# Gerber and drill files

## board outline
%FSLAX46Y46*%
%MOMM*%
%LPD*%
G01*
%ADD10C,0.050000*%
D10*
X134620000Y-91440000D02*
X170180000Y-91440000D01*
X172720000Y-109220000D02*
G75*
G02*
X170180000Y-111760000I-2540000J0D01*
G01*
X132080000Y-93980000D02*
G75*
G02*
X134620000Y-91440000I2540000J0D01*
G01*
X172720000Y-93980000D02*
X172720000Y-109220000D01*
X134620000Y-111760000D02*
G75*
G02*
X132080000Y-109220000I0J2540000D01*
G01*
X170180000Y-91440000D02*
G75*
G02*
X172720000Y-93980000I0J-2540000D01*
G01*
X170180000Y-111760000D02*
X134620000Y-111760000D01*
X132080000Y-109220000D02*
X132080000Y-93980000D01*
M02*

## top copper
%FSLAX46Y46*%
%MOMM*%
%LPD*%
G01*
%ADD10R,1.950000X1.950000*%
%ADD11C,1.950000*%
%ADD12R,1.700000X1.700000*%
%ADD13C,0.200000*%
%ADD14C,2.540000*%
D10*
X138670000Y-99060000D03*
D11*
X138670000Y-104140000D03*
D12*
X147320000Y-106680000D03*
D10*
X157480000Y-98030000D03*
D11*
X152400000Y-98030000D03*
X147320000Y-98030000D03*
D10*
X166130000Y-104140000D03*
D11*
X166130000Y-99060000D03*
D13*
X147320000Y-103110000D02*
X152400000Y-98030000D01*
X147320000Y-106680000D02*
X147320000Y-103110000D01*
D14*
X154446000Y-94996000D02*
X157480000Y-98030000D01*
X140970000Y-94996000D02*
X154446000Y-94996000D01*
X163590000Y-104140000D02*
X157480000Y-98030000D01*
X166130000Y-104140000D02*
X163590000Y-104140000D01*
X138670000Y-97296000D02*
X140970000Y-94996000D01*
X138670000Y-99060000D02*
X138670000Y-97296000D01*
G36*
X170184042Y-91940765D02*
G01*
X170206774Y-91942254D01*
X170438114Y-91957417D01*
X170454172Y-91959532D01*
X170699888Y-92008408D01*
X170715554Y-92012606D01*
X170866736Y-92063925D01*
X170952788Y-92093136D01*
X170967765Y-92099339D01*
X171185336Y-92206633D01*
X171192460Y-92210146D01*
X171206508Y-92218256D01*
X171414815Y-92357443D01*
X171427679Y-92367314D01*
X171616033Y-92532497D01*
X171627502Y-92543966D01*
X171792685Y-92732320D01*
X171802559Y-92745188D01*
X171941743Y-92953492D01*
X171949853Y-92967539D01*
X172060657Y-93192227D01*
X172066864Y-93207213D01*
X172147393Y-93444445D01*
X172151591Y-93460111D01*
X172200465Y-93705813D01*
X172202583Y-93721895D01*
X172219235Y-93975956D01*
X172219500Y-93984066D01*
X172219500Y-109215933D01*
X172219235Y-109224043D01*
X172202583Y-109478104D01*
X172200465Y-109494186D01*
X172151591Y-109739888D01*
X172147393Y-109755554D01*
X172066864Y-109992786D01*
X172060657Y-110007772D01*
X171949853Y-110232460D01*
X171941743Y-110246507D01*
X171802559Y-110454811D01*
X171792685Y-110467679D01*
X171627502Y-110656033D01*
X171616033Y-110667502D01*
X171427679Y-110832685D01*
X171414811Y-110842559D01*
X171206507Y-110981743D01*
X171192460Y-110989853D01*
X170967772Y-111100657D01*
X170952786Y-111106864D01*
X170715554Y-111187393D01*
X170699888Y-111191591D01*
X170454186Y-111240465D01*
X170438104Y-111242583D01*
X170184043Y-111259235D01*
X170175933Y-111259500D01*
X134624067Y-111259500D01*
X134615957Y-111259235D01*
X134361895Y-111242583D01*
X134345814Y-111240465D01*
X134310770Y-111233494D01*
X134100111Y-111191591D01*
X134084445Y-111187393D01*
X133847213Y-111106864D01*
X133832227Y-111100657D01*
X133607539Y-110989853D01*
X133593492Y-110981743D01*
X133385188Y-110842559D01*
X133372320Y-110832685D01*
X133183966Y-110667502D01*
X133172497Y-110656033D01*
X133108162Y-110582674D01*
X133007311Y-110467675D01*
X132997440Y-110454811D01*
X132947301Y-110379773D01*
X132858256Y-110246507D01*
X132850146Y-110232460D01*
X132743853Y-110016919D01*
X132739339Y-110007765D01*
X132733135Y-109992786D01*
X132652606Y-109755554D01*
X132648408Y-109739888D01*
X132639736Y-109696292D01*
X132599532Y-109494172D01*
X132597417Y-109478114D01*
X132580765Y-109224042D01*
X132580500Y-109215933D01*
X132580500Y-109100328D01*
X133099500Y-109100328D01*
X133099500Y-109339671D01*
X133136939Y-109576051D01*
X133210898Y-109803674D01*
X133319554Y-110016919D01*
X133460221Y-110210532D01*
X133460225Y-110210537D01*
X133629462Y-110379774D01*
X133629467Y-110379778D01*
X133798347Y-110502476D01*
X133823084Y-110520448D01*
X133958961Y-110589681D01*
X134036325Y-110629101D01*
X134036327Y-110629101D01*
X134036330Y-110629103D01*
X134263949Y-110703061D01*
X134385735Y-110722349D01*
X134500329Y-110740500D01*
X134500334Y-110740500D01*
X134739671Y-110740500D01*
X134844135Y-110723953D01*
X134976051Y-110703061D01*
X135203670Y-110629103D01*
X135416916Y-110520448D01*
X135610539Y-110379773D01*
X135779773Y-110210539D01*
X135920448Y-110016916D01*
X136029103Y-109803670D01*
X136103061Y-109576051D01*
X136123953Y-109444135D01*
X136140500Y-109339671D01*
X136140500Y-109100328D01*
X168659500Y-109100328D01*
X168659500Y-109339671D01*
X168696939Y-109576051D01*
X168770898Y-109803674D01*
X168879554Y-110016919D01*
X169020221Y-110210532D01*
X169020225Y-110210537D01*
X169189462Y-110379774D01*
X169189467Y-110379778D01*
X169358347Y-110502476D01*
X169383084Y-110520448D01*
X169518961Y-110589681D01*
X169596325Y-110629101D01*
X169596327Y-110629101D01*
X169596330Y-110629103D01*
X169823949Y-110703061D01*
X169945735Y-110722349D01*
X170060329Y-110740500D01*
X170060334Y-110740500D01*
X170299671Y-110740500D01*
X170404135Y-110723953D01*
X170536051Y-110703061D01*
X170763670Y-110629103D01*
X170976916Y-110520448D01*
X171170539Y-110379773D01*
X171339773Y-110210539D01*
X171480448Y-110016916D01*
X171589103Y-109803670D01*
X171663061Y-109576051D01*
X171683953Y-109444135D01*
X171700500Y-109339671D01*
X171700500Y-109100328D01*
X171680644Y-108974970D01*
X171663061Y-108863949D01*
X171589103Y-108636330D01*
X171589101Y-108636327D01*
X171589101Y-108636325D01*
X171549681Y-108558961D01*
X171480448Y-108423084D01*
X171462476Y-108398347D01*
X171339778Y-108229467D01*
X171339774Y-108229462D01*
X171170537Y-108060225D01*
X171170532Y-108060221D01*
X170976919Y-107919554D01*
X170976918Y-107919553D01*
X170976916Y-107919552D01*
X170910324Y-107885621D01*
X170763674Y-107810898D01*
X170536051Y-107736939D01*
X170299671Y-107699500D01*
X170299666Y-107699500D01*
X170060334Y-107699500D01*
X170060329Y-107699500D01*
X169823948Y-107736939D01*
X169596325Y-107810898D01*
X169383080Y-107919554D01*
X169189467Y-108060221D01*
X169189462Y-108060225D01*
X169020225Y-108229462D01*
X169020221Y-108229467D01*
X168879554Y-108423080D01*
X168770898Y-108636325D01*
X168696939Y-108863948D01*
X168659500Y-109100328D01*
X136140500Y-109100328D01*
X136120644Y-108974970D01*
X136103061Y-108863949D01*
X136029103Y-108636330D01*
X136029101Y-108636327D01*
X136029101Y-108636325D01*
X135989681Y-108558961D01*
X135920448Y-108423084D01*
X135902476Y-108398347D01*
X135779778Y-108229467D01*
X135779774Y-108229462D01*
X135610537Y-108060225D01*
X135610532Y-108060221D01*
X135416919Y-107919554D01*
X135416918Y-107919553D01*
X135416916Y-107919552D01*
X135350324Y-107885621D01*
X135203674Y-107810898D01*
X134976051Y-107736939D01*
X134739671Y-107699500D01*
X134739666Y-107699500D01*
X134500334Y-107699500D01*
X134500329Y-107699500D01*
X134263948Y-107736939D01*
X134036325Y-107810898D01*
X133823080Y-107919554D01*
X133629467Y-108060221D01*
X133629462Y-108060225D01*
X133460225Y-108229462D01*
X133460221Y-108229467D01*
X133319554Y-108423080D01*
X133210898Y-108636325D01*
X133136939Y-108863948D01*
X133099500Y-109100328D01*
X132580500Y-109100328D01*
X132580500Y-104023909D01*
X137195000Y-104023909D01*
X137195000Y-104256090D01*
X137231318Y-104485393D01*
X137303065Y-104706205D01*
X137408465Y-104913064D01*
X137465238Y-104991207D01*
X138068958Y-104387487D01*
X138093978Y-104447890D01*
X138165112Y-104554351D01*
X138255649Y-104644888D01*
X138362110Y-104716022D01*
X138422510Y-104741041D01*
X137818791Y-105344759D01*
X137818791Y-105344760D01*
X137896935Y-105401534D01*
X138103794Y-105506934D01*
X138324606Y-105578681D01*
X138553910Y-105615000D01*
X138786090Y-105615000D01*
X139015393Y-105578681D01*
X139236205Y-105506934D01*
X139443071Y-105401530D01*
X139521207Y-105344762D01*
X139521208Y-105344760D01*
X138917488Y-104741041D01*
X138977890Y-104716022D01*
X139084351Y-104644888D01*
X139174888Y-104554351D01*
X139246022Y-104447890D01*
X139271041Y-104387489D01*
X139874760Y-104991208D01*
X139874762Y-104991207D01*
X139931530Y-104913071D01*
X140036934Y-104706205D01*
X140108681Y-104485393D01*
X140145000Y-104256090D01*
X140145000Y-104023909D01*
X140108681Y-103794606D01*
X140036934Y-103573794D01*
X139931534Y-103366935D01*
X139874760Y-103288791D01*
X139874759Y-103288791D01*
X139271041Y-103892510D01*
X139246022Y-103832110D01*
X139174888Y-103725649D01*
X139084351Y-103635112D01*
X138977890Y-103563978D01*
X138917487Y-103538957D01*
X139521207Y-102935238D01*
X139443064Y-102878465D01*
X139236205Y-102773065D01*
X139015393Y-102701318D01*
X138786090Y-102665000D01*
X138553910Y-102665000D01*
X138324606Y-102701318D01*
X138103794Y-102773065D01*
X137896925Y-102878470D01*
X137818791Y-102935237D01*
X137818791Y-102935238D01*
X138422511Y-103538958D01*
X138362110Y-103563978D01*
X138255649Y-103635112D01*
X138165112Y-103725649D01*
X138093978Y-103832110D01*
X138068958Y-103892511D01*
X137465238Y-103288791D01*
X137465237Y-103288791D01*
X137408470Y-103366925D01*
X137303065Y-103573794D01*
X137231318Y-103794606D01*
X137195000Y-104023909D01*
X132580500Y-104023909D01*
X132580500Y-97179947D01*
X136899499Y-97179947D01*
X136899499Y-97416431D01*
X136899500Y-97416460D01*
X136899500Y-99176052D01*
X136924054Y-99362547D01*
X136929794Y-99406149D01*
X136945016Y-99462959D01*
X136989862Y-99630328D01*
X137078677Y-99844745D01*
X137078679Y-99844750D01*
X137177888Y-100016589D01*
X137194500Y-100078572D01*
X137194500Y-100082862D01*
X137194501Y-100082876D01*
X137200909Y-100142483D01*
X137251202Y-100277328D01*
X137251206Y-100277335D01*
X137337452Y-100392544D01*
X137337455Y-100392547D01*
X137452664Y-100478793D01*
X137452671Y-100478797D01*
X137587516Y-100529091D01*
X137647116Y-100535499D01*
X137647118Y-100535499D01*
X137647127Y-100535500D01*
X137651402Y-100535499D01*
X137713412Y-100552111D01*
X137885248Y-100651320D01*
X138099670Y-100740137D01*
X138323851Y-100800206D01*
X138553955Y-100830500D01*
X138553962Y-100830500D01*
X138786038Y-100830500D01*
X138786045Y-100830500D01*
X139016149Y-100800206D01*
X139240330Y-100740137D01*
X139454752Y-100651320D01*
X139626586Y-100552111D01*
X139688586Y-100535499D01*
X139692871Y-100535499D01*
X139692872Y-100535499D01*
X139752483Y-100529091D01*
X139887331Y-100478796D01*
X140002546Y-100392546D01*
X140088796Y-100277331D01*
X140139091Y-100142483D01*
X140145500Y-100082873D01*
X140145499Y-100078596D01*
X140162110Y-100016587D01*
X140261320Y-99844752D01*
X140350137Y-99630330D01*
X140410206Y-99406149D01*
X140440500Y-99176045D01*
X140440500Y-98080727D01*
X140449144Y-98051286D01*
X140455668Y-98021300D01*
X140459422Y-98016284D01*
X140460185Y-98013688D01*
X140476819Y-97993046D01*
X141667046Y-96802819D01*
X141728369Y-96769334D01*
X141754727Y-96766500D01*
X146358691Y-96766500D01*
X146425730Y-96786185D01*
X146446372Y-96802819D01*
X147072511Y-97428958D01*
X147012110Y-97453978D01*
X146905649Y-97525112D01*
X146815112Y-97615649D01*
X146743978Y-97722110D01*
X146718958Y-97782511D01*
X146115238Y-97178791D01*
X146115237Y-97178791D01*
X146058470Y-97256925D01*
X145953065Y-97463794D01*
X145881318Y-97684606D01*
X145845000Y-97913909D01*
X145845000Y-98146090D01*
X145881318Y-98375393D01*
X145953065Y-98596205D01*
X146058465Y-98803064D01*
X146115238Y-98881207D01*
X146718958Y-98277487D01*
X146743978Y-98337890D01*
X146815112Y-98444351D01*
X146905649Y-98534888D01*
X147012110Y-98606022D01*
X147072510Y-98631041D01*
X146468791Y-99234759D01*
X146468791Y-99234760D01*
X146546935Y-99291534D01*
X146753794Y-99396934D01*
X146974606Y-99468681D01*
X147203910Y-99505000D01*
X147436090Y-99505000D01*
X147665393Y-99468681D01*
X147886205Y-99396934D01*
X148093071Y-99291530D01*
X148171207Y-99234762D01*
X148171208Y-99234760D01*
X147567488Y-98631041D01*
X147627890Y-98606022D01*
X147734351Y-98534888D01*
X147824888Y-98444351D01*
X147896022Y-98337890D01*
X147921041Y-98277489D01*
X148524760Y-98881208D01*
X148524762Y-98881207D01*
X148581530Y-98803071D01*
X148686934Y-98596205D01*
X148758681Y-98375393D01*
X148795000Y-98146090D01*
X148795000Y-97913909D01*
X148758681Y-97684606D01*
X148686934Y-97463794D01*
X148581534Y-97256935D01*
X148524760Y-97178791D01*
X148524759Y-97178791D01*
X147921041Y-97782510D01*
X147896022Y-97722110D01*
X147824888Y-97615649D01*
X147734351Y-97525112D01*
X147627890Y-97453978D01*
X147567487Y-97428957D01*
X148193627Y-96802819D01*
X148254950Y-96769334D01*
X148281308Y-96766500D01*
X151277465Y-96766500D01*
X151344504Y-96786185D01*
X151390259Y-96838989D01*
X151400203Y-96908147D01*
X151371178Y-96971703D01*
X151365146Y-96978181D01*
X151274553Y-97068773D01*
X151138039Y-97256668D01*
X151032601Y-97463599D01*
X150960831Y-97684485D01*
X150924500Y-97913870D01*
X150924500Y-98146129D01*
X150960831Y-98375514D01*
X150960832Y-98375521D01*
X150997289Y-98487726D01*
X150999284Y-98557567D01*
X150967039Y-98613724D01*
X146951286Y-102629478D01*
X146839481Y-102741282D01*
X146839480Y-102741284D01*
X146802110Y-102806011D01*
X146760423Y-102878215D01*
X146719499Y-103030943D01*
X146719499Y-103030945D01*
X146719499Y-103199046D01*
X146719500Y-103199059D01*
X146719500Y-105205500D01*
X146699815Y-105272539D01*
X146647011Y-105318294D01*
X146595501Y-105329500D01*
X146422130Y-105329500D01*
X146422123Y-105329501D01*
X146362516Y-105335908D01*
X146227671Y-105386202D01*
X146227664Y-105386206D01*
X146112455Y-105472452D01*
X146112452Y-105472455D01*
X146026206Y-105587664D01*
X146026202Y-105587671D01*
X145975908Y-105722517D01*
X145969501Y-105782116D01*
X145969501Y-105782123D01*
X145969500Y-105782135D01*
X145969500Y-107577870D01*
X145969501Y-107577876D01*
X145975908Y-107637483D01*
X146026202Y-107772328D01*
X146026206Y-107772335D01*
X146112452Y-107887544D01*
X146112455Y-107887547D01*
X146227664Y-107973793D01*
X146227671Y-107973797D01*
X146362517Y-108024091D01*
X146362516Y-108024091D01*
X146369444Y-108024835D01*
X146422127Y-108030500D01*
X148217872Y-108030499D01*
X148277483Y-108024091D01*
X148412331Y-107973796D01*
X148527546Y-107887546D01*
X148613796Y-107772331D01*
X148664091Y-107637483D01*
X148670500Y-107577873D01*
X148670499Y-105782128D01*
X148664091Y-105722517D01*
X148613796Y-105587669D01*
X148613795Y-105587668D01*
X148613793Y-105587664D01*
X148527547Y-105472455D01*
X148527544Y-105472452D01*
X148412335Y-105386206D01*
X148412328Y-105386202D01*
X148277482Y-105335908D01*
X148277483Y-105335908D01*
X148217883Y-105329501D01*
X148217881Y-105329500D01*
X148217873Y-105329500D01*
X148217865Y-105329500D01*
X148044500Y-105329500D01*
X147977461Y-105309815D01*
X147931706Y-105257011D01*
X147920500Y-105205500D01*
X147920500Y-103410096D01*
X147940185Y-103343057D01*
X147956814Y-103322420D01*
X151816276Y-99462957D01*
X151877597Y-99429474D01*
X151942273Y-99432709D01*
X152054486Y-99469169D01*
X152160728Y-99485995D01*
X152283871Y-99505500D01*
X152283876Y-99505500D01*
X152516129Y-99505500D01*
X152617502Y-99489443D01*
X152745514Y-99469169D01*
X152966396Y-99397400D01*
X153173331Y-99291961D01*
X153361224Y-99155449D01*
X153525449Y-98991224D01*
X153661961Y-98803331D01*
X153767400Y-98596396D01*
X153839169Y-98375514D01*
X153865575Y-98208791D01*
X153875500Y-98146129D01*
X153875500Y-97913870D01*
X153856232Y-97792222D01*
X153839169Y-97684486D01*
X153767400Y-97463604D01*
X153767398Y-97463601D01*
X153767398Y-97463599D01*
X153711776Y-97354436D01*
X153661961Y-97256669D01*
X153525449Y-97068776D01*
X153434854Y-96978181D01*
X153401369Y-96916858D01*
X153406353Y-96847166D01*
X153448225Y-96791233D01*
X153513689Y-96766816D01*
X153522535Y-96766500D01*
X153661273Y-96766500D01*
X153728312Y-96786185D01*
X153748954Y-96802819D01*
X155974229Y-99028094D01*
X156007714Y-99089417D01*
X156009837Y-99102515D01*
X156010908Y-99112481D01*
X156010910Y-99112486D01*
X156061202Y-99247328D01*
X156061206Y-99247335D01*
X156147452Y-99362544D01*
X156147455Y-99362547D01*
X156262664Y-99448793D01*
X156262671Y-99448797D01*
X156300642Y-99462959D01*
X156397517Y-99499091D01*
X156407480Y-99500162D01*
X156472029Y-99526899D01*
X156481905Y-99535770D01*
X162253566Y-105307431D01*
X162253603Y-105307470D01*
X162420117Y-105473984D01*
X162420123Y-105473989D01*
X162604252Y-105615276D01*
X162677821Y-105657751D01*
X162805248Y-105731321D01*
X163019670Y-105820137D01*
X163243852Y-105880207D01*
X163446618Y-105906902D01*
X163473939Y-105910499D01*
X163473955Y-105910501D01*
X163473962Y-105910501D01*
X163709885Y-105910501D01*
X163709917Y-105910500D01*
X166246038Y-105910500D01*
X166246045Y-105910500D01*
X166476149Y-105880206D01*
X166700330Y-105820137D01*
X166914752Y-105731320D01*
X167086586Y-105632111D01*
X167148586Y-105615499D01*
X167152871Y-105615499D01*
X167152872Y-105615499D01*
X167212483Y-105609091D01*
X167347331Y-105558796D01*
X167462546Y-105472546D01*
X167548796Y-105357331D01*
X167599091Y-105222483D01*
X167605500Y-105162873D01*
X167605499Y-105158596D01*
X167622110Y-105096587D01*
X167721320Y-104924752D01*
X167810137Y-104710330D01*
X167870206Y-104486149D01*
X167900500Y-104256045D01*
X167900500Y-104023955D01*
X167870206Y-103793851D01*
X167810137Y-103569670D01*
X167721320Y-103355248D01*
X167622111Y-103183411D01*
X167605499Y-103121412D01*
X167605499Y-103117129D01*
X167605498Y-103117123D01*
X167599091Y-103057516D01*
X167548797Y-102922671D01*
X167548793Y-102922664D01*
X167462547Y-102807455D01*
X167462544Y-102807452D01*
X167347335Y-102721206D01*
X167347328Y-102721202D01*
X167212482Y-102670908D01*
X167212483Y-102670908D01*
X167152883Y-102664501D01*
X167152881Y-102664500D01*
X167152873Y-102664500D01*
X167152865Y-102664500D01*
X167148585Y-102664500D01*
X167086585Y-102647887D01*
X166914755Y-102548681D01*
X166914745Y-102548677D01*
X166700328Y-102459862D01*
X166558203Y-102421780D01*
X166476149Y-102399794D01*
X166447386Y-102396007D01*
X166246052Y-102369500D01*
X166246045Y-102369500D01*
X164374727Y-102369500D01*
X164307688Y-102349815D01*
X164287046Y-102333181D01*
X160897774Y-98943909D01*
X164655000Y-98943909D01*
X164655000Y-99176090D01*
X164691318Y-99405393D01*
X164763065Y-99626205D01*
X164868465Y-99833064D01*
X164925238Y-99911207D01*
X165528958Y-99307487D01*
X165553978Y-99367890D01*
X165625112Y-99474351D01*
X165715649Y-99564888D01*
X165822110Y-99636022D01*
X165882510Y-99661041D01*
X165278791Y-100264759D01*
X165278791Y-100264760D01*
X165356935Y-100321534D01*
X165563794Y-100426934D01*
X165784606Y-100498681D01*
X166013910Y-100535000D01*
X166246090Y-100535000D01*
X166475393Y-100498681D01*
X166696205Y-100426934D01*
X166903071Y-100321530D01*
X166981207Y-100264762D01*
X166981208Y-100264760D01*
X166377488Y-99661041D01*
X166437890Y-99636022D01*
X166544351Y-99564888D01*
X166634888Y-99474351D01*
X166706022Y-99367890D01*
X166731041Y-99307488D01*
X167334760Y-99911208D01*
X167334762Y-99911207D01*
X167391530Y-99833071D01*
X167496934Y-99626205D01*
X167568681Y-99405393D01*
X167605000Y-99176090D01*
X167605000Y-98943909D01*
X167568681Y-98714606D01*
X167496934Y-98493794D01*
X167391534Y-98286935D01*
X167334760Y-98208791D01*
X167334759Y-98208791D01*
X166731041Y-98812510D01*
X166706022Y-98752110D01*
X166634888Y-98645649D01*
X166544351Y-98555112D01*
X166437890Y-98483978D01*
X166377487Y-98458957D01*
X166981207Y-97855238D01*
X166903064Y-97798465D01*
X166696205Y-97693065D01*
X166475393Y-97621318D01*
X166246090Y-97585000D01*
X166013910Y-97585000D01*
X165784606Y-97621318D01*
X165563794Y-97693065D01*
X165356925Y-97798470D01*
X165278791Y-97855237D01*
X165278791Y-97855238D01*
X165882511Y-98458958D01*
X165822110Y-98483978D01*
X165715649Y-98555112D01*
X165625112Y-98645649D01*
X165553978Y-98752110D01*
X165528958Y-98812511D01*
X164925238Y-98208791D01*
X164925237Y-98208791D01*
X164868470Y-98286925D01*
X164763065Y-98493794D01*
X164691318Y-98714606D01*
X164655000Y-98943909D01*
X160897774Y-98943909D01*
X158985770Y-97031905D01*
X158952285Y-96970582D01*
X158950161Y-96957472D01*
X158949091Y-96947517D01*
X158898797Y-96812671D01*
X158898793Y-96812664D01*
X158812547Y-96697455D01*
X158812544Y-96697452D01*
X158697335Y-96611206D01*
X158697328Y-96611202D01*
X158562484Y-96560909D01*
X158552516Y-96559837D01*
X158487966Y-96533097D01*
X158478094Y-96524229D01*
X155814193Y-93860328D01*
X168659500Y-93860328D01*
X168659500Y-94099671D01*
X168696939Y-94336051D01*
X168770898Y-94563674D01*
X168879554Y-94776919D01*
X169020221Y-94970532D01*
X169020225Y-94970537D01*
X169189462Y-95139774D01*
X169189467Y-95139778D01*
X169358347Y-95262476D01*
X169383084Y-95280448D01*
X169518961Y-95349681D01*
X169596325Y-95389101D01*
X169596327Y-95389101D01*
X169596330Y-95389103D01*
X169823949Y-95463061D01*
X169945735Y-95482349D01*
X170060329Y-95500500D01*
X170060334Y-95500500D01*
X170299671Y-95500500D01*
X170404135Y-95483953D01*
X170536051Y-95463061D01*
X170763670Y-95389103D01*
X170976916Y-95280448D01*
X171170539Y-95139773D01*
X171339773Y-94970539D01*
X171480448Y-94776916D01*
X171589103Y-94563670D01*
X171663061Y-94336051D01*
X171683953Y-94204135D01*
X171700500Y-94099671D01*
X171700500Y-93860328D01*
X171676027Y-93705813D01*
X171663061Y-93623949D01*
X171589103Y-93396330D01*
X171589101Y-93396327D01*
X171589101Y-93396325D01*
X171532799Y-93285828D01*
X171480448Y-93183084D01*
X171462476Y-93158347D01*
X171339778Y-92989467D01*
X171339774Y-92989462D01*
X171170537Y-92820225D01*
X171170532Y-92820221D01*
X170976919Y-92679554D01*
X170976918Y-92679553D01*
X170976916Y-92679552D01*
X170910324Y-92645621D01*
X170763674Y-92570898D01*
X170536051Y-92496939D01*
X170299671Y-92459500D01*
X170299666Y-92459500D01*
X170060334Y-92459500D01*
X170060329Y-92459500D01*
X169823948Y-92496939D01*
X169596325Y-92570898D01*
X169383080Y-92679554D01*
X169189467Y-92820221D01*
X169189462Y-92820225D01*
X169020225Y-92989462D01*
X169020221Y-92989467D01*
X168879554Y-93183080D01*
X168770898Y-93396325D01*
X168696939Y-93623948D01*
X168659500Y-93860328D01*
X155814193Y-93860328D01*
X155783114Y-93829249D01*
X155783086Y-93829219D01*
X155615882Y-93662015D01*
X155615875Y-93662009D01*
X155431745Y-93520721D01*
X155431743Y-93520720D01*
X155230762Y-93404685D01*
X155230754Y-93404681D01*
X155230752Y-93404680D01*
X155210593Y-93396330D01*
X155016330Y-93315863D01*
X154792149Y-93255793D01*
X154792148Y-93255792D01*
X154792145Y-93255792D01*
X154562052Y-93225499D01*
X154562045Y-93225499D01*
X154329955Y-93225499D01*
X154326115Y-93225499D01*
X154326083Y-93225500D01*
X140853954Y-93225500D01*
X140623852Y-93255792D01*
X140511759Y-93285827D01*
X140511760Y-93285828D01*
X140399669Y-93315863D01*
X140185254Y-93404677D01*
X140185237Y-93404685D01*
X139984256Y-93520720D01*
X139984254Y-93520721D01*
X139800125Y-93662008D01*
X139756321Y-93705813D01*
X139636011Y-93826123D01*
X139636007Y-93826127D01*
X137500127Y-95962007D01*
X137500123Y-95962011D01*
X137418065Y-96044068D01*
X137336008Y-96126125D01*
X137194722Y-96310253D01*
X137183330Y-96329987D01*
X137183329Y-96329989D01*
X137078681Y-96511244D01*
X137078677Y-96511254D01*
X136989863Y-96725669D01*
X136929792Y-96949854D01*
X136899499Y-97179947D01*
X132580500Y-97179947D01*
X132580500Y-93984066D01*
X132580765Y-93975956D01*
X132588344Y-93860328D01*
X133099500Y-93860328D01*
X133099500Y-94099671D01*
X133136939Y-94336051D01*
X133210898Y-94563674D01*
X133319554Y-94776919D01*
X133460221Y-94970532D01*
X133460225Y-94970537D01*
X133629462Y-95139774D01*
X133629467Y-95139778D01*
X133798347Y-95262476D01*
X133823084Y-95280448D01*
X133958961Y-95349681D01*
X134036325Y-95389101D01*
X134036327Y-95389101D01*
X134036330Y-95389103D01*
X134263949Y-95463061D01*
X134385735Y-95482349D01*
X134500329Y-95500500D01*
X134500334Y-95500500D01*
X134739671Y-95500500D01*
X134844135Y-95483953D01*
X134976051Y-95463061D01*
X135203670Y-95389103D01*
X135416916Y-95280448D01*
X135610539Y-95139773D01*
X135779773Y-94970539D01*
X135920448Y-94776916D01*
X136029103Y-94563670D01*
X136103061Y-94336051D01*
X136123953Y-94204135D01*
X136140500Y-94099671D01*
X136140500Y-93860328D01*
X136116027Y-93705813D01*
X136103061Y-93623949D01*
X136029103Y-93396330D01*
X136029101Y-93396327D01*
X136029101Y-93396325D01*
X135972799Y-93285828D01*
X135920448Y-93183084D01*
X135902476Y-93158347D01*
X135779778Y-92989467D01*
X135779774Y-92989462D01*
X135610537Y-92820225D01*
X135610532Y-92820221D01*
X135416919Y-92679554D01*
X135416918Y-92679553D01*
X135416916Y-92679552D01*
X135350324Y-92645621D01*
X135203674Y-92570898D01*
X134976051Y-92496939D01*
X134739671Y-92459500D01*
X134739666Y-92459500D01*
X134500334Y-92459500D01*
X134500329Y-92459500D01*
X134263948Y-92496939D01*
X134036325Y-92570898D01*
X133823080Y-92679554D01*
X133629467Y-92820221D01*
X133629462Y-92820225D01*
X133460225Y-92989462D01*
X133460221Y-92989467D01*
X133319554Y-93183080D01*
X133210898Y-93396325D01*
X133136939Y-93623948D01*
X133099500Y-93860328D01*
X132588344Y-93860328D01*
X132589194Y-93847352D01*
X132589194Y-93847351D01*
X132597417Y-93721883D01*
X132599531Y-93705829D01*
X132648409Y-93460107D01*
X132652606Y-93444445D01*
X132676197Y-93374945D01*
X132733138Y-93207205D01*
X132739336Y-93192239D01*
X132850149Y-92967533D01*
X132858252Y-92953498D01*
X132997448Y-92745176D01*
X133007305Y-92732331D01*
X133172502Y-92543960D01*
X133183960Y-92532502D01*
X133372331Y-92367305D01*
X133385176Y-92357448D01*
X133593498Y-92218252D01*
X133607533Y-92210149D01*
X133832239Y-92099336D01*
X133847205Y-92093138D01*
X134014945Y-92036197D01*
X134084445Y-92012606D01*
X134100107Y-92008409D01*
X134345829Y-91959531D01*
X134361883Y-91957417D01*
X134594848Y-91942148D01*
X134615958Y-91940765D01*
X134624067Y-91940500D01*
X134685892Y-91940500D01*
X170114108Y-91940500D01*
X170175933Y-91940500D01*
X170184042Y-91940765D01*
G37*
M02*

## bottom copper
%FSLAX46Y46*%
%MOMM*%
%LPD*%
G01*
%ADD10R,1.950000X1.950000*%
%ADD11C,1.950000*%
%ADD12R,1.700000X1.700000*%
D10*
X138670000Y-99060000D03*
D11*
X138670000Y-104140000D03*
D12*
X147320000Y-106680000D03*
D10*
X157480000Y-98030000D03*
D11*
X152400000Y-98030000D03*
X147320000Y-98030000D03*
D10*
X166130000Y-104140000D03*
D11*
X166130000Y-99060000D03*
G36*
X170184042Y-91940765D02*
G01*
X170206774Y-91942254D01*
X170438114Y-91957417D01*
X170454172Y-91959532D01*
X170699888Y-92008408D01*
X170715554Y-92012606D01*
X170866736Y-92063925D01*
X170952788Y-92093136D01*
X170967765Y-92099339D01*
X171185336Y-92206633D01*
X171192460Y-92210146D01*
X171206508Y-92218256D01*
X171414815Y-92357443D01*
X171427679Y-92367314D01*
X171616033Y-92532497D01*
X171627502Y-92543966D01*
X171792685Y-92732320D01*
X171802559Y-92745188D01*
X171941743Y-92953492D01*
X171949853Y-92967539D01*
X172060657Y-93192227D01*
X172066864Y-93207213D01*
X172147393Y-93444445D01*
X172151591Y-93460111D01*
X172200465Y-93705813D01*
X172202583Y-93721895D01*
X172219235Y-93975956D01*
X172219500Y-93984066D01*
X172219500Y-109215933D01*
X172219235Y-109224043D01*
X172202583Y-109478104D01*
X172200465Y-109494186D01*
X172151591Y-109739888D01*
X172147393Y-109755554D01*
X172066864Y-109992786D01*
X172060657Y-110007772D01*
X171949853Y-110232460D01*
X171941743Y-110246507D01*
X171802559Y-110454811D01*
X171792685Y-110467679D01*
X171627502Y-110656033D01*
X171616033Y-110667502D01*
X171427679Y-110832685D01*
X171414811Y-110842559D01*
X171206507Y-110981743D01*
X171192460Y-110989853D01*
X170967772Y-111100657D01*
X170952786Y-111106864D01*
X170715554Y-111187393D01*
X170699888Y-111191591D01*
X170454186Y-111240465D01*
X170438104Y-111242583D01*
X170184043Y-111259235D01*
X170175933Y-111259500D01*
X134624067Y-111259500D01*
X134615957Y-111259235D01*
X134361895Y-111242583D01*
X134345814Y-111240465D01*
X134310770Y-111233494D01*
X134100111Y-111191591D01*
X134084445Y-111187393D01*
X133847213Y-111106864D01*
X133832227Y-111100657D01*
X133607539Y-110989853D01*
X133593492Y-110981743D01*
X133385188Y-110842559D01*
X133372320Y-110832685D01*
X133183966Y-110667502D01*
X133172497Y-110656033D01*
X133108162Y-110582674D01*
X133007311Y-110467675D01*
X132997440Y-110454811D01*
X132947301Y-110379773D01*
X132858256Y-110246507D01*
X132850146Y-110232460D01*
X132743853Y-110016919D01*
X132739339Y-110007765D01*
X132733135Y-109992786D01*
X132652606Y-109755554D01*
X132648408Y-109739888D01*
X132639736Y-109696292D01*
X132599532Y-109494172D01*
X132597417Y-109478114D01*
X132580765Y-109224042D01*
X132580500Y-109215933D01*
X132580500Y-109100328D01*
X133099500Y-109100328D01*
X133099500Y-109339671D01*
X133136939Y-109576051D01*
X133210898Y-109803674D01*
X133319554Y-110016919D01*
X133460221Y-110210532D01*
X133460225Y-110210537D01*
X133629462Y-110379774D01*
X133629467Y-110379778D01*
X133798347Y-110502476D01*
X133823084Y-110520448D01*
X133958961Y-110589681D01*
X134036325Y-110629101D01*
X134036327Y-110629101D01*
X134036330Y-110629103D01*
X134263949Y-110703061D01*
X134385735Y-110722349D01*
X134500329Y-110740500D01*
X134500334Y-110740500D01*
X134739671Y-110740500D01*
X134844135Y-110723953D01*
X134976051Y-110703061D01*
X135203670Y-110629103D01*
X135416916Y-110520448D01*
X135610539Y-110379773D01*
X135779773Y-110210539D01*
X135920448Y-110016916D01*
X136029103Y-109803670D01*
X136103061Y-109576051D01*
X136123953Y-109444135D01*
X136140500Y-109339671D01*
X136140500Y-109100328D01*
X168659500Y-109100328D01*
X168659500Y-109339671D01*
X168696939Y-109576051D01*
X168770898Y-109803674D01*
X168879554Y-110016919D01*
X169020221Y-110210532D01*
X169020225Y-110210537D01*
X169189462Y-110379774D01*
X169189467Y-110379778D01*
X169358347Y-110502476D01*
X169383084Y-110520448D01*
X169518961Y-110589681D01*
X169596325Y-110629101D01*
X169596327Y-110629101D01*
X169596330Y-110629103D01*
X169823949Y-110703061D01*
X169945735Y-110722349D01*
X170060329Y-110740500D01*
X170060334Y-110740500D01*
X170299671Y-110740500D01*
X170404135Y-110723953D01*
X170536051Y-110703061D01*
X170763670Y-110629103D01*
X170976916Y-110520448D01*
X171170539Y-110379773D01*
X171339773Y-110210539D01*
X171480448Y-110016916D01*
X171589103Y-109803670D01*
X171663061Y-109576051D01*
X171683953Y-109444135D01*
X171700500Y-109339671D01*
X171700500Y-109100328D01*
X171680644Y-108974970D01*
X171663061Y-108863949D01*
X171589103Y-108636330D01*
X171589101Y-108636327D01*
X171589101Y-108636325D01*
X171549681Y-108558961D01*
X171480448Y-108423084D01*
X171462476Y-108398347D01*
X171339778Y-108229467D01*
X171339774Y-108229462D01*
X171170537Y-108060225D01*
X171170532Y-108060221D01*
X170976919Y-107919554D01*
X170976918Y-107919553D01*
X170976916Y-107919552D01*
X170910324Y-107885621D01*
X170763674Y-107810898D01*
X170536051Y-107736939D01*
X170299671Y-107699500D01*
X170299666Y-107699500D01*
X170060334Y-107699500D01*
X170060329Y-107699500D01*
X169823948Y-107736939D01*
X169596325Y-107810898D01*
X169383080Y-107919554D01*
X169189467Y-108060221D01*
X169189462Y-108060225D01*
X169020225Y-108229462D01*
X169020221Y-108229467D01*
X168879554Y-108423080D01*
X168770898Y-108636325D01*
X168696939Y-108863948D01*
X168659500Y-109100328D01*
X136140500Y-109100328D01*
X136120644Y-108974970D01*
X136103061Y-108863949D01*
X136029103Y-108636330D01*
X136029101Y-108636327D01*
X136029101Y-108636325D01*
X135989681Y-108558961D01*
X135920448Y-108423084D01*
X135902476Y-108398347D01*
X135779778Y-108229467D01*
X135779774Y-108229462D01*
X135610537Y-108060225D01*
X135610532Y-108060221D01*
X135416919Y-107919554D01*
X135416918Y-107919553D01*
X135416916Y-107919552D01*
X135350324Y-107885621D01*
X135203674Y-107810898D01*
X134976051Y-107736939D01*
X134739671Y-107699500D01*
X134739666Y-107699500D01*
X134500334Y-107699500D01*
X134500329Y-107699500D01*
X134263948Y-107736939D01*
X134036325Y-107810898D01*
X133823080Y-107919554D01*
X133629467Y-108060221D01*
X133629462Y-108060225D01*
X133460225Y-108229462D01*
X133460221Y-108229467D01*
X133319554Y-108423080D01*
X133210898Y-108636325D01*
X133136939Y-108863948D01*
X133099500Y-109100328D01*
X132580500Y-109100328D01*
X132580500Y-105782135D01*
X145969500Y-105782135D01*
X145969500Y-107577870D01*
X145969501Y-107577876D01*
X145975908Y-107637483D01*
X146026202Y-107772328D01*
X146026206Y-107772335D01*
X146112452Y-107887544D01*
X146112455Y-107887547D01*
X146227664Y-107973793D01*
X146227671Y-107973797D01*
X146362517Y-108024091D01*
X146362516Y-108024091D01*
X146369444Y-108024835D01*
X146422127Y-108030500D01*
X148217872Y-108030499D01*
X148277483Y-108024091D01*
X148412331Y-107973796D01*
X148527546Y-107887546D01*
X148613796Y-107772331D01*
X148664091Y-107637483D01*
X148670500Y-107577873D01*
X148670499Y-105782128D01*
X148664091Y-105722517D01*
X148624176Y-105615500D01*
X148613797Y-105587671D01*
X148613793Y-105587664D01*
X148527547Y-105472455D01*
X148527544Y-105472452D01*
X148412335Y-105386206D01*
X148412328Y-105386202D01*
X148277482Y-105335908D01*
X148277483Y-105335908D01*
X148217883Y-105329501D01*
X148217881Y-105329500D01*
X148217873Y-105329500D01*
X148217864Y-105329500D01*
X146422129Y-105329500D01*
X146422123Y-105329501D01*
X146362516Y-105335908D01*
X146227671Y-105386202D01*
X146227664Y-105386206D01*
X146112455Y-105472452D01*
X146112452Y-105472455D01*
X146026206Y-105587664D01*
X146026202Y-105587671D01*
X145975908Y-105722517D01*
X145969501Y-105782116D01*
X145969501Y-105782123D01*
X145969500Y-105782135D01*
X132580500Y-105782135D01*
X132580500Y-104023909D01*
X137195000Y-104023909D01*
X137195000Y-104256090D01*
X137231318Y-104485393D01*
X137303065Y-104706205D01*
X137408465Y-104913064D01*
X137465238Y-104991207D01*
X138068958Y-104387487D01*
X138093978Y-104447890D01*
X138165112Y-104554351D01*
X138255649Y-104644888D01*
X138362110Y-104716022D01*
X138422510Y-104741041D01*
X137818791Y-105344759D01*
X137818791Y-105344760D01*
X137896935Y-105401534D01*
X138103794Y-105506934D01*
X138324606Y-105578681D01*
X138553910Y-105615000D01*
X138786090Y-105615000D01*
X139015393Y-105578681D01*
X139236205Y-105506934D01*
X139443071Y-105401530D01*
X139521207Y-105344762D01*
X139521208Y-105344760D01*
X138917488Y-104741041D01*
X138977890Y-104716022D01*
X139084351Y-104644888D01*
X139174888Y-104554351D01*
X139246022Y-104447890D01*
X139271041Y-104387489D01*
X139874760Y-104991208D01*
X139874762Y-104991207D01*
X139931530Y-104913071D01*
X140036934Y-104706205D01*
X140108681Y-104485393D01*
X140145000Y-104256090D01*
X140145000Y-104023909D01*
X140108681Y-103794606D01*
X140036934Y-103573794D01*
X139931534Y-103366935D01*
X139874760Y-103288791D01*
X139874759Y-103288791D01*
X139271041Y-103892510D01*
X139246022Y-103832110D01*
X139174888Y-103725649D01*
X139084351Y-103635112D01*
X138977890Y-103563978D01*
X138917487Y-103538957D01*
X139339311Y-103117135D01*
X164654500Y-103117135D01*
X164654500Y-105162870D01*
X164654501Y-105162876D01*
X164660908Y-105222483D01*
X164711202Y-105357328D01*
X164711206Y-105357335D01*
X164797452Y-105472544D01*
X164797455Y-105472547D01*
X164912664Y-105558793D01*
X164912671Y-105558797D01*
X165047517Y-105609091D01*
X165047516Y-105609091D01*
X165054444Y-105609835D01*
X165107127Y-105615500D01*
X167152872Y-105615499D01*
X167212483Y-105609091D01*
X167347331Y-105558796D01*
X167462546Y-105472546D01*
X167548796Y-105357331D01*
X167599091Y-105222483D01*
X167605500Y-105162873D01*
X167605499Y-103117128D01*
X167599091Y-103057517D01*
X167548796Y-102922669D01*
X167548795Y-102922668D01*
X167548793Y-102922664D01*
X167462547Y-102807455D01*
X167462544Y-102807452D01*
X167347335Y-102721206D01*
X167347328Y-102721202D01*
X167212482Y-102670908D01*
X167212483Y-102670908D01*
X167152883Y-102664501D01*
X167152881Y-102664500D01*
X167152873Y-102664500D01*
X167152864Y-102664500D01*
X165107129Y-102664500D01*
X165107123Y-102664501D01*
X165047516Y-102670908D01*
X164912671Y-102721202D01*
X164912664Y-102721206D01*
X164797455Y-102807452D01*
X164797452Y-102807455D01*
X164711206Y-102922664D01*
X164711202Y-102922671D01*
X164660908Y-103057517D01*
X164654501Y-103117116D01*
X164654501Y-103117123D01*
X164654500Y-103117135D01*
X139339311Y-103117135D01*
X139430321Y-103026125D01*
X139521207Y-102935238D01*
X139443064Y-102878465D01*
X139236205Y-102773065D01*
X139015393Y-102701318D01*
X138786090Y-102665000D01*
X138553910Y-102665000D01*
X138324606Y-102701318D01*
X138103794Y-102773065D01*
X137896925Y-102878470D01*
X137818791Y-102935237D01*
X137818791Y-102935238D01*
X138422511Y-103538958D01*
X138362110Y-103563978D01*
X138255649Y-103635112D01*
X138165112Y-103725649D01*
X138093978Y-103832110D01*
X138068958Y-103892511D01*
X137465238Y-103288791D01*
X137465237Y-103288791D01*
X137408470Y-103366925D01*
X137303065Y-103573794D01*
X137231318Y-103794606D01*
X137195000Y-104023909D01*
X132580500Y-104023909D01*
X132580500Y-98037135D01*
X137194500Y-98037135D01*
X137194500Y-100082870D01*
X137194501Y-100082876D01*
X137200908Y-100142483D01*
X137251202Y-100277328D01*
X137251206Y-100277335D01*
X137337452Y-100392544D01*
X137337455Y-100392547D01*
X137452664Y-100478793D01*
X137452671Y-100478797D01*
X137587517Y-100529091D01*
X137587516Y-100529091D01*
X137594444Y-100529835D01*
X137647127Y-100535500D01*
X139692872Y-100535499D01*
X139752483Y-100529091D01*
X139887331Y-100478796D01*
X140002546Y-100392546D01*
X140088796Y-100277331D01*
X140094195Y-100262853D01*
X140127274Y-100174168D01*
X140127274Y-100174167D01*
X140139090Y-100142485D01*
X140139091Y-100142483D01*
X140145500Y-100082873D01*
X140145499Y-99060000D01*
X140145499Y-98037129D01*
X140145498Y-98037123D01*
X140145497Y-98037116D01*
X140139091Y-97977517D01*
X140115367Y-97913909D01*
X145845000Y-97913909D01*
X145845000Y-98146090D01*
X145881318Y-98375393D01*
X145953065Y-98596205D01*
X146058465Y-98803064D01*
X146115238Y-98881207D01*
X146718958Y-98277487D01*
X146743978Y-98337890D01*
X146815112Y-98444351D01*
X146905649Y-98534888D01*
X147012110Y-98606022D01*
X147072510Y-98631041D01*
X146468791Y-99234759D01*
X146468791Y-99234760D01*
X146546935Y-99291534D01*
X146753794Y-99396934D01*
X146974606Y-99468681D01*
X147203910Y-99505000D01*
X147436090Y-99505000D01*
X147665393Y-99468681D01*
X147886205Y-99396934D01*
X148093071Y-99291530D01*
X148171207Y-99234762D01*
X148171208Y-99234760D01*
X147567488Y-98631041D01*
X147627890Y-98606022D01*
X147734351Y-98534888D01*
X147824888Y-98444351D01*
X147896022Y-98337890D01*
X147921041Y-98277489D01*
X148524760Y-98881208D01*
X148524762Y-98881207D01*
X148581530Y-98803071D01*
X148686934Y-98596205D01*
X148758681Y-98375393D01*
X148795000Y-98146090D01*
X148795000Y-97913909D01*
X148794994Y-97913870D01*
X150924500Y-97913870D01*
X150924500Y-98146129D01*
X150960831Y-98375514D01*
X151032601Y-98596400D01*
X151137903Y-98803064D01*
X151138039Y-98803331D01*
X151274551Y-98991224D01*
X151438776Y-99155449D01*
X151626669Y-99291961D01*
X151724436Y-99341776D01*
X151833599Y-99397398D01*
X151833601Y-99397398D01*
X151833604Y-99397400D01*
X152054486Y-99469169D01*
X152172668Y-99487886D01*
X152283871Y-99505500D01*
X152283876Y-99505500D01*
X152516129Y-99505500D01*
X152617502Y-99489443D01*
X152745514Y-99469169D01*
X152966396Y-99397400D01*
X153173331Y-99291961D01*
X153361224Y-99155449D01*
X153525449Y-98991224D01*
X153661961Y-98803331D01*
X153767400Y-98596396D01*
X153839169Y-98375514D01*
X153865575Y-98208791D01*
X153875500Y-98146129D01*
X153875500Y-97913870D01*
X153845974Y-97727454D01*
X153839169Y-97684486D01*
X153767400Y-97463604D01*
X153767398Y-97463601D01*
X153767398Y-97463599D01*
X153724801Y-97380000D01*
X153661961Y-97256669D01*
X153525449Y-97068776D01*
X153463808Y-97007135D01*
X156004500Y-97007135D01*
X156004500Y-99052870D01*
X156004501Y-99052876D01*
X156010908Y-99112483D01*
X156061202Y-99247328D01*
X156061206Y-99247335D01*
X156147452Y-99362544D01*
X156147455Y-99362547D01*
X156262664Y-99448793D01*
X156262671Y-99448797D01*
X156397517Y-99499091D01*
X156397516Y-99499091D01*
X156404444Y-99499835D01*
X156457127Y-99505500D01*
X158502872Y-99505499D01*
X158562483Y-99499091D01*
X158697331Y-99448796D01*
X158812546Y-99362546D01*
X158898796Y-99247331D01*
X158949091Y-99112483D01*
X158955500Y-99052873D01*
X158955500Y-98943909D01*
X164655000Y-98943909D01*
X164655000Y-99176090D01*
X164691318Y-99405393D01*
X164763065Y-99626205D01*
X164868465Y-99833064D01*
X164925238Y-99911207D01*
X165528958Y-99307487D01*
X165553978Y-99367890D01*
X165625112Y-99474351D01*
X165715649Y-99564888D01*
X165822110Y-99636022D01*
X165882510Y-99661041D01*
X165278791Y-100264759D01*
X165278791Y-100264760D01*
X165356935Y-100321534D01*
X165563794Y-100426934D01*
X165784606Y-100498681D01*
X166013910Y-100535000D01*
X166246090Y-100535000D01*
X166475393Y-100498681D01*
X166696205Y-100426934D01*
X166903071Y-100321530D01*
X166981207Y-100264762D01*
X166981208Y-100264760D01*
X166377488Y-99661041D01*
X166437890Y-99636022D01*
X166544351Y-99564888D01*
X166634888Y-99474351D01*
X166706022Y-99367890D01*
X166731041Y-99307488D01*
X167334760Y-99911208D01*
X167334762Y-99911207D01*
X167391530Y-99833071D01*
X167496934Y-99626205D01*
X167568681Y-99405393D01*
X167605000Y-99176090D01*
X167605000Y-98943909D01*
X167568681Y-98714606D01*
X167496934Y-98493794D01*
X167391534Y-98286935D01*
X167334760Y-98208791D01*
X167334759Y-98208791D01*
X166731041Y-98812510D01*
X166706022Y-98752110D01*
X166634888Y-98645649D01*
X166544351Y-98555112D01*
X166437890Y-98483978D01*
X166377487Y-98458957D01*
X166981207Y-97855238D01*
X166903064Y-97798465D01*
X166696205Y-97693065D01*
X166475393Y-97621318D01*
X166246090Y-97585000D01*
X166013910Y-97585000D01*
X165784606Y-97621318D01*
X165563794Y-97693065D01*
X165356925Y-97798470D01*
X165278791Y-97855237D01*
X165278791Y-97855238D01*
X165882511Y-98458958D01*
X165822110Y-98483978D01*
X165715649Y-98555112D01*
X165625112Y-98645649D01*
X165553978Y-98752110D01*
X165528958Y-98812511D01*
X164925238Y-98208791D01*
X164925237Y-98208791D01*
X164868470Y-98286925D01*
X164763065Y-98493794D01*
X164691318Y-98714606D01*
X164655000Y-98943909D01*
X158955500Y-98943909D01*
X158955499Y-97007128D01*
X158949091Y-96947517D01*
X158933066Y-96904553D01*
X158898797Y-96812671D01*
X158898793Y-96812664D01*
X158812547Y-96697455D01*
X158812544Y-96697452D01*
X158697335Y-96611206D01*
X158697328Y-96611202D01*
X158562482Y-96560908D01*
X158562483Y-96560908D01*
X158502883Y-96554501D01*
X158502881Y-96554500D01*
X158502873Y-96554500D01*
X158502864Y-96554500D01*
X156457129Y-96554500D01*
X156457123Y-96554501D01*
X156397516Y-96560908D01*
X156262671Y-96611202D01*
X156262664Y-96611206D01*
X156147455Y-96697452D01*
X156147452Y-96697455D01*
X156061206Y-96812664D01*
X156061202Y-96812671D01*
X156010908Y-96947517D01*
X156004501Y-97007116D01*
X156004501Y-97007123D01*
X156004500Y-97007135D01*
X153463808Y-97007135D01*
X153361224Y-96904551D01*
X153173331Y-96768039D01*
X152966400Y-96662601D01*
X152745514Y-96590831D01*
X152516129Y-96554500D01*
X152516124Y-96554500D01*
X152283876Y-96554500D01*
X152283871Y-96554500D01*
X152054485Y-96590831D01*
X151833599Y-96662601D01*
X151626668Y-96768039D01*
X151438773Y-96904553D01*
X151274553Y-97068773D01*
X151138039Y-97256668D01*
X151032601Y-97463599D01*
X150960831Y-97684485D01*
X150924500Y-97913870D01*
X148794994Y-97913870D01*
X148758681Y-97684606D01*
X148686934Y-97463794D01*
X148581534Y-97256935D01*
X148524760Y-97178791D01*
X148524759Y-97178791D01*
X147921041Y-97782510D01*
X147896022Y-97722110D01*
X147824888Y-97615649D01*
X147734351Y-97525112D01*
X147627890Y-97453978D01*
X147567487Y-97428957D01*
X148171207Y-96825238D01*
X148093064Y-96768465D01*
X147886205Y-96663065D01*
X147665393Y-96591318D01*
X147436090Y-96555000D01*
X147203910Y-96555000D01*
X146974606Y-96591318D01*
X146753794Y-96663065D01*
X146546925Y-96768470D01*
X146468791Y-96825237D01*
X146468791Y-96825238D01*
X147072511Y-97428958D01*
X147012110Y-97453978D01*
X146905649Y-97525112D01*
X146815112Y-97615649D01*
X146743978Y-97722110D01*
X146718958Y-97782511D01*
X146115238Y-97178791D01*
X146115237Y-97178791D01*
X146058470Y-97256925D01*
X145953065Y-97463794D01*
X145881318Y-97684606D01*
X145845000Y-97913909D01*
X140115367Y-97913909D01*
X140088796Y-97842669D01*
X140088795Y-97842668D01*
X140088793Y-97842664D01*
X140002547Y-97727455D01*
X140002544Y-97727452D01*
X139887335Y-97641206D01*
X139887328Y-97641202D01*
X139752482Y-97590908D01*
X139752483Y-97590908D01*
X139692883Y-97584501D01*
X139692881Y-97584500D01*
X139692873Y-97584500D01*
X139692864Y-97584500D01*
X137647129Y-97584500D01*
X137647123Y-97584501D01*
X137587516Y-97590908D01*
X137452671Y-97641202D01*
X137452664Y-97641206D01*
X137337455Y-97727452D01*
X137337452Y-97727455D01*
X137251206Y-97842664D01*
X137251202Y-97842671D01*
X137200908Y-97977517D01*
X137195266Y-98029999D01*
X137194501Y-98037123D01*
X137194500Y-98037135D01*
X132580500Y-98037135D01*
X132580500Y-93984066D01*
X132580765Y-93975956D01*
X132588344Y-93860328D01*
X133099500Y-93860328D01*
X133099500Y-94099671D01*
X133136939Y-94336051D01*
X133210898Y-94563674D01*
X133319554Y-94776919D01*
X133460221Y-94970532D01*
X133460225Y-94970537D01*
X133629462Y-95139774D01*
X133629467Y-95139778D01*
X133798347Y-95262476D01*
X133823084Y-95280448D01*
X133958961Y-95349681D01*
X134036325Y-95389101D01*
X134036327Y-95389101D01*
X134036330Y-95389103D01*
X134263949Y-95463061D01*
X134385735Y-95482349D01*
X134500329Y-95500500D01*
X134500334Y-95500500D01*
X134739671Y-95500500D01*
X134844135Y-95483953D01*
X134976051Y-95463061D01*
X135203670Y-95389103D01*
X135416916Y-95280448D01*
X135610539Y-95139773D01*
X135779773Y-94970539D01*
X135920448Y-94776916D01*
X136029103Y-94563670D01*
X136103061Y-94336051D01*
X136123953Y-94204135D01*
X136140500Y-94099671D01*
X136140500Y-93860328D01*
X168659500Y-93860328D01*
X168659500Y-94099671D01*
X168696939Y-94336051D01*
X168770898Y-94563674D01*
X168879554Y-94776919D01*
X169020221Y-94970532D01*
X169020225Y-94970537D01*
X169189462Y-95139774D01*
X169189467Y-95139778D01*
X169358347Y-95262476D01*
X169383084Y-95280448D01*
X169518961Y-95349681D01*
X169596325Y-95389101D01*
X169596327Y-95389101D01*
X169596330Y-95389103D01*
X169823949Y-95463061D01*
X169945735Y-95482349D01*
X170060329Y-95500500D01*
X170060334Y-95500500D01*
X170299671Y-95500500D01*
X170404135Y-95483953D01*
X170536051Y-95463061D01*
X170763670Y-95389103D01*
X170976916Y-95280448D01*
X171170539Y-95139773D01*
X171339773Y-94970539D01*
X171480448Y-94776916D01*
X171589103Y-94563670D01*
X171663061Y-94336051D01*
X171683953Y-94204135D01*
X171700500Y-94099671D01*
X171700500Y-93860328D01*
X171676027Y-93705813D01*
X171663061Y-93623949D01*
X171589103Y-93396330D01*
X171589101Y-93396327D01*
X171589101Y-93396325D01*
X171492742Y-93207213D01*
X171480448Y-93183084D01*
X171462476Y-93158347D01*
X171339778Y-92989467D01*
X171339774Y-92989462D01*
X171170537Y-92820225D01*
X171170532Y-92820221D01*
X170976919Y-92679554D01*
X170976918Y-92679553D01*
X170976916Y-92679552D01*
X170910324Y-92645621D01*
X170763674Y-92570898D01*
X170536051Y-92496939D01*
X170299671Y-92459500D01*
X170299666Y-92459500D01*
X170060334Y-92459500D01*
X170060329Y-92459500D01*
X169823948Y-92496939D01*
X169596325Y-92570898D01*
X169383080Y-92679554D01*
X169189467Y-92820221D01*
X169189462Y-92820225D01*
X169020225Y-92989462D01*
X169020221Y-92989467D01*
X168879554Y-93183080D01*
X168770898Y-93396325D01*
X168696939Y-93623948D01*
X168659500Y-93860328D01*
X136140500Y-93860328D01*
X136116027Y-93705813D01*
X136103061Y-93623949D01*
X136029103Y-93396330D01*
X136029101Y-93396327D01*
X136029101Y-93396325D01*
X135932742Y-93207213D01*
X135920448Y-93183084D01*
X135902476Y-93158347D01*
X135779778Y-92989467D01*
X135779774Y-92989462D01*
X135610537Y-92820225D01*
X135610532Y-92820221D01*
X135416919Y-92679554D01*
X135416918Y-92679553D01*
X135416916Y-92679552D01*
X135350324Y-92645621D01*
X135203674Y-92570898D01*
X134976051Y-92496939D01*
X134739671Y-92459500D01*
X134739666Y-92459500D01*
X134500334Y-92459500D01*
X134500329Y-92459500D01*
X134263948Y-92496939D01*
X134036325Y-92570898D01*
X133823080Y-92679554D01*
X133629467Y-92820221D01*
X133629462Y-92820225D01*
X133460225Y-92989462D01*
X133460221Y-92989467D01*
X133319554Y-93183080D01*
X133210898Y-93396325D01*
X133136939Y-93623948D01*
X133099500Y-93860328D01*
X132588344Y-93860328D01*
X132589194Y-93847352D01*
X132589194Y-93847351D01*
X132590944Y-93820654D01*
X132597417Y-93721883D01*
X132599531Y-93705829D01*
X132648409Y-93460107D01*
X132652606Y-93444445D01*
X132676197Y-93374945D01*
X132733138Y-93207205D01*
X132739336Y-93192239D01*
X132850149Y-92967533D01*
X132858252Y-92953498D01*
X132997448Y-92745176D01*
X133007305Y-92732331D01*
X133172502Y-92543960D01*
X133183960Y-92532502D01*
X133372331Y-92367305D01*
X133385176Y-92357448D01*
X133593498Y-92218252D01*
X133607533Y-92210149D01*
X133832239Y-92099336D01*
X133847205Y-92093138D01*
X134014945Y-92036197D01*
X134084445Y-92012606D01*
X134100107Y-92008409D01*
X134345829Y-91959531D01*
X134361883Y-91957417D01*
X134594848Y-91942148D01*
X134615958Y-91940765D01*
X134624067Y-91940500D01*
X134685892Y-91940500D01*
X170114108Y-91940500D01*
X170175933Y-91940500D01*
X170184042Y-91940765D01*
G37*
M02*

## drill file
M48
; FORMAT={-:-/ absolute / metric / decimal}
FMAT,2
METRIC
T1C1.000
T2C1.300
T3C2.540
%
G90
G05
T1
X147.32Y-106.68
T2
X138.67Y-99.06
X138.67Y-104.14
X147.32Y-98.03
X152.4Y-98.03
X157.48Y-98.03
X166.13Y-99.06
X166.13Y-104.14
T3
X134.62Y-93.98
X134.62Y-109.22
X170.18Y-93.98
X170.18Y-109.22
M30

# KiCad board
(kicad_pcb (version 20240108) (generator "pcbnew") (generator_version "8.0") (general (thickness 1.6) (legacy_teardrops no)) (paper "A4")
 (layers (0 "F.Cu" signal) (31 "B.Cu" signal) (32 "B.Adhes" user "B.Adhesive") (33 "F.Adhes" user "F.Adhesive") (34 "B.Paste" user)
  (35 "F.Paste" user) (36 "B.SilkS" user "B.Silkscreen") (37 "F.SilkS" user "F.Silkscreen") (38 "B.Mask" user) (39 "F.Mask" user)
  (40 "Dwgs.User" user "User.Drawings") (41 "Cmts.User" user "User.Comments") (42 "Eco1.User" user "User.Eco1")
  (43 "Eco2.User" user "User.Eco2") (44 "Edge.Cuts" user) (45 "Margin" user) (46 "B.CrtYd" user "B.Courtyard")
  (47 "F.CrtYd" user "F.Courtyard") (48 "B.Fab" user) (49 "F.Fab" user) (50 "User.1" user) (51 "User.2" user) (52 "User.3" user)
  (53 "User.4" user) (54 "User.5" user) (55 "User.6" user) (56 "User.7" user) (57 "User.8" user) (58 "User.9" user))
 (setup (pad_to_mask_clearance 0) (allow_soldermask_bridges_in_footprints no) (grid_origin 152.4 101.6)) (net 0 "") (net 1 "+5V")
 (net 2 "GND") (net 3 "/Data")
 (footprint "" (layer "F.Cu") (at 134.62 109.22)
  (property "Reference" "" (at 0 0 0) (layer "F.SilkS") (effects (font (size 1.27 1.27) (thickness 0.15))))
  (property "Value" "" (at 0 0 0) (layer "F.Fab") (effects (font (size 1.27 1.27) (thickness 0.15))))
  (pad "" np_thru_hole circle (at 0 0) (size 2.5 2.5) (drill 2.54) (layers "F&B.Cu" "*.Mask")))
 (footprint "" (layer "F.Cu") (at 170.18 93.98)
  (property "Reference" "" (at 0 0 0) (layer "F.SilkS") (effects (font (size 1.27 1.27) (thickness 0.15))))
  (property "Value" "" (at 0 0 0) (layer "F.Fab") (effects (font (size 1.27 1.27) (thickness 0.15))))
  (pad "" np_thru_hole circle (at 0 0) (size 2.5 2.5) (drill 2.54) (layers "F&B.Cu" "*.Mask")))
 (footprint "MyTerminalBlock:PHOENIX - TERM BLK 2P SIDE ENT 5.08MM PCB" (layer "F.Cu") (at 134.62 96.52 -90)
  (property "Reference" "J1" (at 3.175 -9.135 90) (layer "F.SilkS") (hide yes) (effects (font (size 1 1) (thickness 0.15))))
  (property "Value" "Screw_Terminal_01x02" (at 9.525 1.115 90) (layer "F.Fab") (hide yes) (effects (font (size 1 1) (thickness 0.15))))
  (pad "1" thru_hole rect (at 2.54 -4.05 270) (size 1.95 1.95) (drill 1.3) (layers "*.Cu" "*.Mask") (remove_unused_layers no) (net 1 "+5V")
   (solder_mask_margin 0.102))
  (pad "2" thru_hole circle (at 7.62 -4.05 270) (size 1.95 1.95) (drill 1.3) (layers "*.Cu" "*.Mask") (remove_unused_layers no)
   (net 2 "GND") (solder_mask_margin 0.102)))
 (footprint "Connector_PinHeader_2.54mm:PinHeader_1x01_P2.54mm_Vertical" (layer "F.Cu") (at 147.32 106.68 -90)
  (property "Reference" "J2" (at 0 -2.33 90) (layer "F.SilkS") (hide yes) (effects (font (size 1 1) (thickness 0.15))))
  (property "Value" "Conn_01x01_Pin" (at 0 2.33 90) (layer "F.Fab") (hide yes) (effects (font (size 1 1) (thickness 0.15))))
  (pad "1" thru_hole rect (at 0 0 270) (size 1.7 1.7) (drill 1) (layers "*.Cu" "*.Mask") (remove_unused_layers no) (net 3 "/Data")))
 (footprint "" (layer "F.Cu") (at 134.62 93.98)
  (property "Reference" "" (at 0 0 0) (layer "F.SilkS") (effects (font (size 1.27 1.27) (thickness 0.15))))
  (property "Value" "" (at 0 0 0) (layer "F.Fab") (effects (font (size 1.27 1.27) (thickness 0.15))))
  (pad "" np_thru_hole circle (at 0 0) (size 2.5 2.5) (drill 2.54) (layers "F&B.Cu" "*.Mask")))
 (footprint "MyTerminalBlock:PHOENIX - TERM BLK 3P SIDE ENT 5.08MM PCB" (layer "F.Cu") (at 160.02 93.98 180)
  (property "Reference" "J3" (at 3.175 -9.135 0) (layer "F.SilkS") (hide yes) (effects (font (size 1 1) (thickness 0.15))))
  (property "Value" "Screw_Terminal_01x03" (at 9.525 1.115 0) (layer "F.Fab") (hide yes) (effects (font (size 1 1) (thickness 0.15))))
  (pad "1" thru_hole rect (at 2.54 -4.05 180) (size 1.95 1.95) (drill 1.3) (layers "*.Cu" "*.Mask") (remove_unused_layers no) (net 1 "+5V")
   (solder_mask_margin 0.102))
  (pad "2" thru_hole circle (at 7.62 -4.05 180) (size 1.95 1.95) (drill 1.3) (layers "*.Cu" "*.Mask") (remove_unused_layers no)
   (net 3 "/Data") (solder_mask_margin 0.102))
  (pad "3" thru_hole circle (at 12.7 -4.05 180) (size 1.95 1.95) (drill 1.3) (layers "*.Cu" "*.Mask") (remove_unused_layers no)
   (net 2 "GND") (solder_mask_margin 0.102)))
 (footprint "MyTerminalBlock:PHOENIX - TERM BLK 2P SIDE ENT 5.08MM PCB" (layer "F.Cu") (at 170.18 106.68 90)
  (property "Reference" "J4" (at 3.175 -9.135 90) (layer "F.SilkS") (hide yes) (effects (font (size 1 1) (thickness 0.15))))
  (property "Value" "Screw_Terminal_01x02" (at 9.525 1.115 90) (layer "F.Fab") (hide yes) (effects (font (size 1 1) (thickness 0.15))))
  (pad "1" thru_hole rect (at 2.54 -4.05 90) (size 1.95 1.95) (drill 1.3) (layers "*.Cu" "*.Mask") (remove_unused_layers no) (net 1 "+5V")
   (solder_mask_margin 0.102))
  (pad "2" thru_hole circle (at 7.62 -4.05 90) (size 1.95 1.95) (drill 1.3) (layers "*.Cu" "*.Mask") (remove_unused_layers no) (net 2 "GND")
   (solder_mask_margin 0.102)))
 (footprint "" (layer "F.Cu") (at 170.18 109.22)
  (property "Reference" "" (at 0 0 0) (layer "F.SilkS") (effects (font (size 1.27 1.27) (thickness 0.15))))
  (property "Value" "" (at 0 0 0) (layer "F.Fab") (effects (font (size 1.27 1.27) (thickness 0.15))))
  (pad "" np_thru_hole circle (at 0 0) (size 2.5 2.5) (drill 2.54) (layers "F&B.Cu" "*.Mask")))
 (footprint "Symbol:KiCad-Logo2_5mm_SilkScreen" (layer "B.Cu") (at 156.845 106.045 180)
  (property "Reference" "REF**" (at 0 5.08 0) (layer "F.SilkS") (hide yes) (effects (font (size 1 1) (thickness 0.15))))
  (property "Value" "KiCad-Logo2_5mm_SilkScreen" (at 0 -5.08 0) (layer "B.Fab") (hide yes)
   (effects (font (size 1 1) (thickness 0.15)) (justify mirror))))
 (gr_line (start 134.62 91.44) (end 170.18 91.44) (stroke (width 0.05) (type default)) (layer "Edge.Cuts"))
 (gr_arc (start 172.72 109.22) (mid 171.976051 111.016051) (end 170.18 111.76) (stroke (width 0.05) (type default)) (layer "Edge.Cuts"))
 (gr_arc (start 132.08 93.98) (mid 132.823949 92.183949) (end 134.62 91.44) (stroke (width 0.05) (type default)) (layer "Edge.Cuts"))
 (gr_line (start 172.72 93.98) (end 172.72 109.22) (stroke (width 0.05) (type default)) (layer "Edge.Cuts"))
 (gr_arc (start 134.62 111.76) (mid 132.823949 111.016051) (end 132.08 109.22) (stroke (width 0.05) (type default)) (layer "Edge.Cuts"))
 (gr_arc (start 170.18 91.44) (mid 171.976051 92.183949) (end 172.72 93.98) (stroke (width 0.05) (type default)) (layer "Edge.Cuts"))
 (gr_line (start 170.18 111.76) (end 134.62 111.76) (stroke (width 0.05) (type default)) (layer "Edge.Cuts"))
 (gr_line (start 132.08 109.22) (end 132.08 93.98) (stroke (width 0.05) (type default)) (layer "Edge.Cuts"))
 (segment (start 147.32 103.11) (end 152.4 98.03) (width 0.2) (layer "F.Cu") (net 3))
 (segment (start 147.32 106.68) (end 147.32 103.11) (width 0.2) (layer "F.Cu") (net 3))
 (segment (start 154.446 94.996) (end 157.48 98.03) (width 2.54) (layer "F.Cu") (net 1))
 (segment (start 140.97 94.996) (end 154.446 94.996) (width 2.54) (layer "F.Cu") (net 1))
 (segment (start 163.59 104.14) (end 157.48 98.03) (width 2.54) (layer "F.Cu") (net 1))
 (segment (start 166.13 104.14) (end 163.59 104.14) (width 2.54) (layer "F.Cu") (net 1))
 (segment (start 138.67 97.296) (end 140.97 94.996) (width 2.54) (layer "F.Cu") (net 1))
 (segment (start 138.67 99.06) (end 138.67 97.296) (width 2.54) (layer "F.Cu") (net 1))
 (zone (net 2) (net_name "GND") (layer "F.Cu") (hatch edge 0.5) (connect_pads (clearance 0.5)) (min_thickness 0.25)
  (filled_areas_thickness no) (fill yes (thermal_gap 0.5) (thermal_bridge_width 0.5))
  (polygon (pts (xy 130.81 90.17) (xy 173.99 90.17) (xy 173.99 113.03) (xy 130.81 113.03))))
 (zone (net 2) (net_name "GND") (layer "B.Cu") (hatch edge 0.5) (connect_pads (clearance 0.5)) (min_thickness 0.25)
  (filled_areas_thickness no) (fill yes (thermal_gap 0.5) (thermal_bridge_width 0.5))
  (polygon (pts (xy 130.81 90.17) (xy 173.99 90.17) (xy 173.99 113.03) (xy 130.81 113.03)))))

